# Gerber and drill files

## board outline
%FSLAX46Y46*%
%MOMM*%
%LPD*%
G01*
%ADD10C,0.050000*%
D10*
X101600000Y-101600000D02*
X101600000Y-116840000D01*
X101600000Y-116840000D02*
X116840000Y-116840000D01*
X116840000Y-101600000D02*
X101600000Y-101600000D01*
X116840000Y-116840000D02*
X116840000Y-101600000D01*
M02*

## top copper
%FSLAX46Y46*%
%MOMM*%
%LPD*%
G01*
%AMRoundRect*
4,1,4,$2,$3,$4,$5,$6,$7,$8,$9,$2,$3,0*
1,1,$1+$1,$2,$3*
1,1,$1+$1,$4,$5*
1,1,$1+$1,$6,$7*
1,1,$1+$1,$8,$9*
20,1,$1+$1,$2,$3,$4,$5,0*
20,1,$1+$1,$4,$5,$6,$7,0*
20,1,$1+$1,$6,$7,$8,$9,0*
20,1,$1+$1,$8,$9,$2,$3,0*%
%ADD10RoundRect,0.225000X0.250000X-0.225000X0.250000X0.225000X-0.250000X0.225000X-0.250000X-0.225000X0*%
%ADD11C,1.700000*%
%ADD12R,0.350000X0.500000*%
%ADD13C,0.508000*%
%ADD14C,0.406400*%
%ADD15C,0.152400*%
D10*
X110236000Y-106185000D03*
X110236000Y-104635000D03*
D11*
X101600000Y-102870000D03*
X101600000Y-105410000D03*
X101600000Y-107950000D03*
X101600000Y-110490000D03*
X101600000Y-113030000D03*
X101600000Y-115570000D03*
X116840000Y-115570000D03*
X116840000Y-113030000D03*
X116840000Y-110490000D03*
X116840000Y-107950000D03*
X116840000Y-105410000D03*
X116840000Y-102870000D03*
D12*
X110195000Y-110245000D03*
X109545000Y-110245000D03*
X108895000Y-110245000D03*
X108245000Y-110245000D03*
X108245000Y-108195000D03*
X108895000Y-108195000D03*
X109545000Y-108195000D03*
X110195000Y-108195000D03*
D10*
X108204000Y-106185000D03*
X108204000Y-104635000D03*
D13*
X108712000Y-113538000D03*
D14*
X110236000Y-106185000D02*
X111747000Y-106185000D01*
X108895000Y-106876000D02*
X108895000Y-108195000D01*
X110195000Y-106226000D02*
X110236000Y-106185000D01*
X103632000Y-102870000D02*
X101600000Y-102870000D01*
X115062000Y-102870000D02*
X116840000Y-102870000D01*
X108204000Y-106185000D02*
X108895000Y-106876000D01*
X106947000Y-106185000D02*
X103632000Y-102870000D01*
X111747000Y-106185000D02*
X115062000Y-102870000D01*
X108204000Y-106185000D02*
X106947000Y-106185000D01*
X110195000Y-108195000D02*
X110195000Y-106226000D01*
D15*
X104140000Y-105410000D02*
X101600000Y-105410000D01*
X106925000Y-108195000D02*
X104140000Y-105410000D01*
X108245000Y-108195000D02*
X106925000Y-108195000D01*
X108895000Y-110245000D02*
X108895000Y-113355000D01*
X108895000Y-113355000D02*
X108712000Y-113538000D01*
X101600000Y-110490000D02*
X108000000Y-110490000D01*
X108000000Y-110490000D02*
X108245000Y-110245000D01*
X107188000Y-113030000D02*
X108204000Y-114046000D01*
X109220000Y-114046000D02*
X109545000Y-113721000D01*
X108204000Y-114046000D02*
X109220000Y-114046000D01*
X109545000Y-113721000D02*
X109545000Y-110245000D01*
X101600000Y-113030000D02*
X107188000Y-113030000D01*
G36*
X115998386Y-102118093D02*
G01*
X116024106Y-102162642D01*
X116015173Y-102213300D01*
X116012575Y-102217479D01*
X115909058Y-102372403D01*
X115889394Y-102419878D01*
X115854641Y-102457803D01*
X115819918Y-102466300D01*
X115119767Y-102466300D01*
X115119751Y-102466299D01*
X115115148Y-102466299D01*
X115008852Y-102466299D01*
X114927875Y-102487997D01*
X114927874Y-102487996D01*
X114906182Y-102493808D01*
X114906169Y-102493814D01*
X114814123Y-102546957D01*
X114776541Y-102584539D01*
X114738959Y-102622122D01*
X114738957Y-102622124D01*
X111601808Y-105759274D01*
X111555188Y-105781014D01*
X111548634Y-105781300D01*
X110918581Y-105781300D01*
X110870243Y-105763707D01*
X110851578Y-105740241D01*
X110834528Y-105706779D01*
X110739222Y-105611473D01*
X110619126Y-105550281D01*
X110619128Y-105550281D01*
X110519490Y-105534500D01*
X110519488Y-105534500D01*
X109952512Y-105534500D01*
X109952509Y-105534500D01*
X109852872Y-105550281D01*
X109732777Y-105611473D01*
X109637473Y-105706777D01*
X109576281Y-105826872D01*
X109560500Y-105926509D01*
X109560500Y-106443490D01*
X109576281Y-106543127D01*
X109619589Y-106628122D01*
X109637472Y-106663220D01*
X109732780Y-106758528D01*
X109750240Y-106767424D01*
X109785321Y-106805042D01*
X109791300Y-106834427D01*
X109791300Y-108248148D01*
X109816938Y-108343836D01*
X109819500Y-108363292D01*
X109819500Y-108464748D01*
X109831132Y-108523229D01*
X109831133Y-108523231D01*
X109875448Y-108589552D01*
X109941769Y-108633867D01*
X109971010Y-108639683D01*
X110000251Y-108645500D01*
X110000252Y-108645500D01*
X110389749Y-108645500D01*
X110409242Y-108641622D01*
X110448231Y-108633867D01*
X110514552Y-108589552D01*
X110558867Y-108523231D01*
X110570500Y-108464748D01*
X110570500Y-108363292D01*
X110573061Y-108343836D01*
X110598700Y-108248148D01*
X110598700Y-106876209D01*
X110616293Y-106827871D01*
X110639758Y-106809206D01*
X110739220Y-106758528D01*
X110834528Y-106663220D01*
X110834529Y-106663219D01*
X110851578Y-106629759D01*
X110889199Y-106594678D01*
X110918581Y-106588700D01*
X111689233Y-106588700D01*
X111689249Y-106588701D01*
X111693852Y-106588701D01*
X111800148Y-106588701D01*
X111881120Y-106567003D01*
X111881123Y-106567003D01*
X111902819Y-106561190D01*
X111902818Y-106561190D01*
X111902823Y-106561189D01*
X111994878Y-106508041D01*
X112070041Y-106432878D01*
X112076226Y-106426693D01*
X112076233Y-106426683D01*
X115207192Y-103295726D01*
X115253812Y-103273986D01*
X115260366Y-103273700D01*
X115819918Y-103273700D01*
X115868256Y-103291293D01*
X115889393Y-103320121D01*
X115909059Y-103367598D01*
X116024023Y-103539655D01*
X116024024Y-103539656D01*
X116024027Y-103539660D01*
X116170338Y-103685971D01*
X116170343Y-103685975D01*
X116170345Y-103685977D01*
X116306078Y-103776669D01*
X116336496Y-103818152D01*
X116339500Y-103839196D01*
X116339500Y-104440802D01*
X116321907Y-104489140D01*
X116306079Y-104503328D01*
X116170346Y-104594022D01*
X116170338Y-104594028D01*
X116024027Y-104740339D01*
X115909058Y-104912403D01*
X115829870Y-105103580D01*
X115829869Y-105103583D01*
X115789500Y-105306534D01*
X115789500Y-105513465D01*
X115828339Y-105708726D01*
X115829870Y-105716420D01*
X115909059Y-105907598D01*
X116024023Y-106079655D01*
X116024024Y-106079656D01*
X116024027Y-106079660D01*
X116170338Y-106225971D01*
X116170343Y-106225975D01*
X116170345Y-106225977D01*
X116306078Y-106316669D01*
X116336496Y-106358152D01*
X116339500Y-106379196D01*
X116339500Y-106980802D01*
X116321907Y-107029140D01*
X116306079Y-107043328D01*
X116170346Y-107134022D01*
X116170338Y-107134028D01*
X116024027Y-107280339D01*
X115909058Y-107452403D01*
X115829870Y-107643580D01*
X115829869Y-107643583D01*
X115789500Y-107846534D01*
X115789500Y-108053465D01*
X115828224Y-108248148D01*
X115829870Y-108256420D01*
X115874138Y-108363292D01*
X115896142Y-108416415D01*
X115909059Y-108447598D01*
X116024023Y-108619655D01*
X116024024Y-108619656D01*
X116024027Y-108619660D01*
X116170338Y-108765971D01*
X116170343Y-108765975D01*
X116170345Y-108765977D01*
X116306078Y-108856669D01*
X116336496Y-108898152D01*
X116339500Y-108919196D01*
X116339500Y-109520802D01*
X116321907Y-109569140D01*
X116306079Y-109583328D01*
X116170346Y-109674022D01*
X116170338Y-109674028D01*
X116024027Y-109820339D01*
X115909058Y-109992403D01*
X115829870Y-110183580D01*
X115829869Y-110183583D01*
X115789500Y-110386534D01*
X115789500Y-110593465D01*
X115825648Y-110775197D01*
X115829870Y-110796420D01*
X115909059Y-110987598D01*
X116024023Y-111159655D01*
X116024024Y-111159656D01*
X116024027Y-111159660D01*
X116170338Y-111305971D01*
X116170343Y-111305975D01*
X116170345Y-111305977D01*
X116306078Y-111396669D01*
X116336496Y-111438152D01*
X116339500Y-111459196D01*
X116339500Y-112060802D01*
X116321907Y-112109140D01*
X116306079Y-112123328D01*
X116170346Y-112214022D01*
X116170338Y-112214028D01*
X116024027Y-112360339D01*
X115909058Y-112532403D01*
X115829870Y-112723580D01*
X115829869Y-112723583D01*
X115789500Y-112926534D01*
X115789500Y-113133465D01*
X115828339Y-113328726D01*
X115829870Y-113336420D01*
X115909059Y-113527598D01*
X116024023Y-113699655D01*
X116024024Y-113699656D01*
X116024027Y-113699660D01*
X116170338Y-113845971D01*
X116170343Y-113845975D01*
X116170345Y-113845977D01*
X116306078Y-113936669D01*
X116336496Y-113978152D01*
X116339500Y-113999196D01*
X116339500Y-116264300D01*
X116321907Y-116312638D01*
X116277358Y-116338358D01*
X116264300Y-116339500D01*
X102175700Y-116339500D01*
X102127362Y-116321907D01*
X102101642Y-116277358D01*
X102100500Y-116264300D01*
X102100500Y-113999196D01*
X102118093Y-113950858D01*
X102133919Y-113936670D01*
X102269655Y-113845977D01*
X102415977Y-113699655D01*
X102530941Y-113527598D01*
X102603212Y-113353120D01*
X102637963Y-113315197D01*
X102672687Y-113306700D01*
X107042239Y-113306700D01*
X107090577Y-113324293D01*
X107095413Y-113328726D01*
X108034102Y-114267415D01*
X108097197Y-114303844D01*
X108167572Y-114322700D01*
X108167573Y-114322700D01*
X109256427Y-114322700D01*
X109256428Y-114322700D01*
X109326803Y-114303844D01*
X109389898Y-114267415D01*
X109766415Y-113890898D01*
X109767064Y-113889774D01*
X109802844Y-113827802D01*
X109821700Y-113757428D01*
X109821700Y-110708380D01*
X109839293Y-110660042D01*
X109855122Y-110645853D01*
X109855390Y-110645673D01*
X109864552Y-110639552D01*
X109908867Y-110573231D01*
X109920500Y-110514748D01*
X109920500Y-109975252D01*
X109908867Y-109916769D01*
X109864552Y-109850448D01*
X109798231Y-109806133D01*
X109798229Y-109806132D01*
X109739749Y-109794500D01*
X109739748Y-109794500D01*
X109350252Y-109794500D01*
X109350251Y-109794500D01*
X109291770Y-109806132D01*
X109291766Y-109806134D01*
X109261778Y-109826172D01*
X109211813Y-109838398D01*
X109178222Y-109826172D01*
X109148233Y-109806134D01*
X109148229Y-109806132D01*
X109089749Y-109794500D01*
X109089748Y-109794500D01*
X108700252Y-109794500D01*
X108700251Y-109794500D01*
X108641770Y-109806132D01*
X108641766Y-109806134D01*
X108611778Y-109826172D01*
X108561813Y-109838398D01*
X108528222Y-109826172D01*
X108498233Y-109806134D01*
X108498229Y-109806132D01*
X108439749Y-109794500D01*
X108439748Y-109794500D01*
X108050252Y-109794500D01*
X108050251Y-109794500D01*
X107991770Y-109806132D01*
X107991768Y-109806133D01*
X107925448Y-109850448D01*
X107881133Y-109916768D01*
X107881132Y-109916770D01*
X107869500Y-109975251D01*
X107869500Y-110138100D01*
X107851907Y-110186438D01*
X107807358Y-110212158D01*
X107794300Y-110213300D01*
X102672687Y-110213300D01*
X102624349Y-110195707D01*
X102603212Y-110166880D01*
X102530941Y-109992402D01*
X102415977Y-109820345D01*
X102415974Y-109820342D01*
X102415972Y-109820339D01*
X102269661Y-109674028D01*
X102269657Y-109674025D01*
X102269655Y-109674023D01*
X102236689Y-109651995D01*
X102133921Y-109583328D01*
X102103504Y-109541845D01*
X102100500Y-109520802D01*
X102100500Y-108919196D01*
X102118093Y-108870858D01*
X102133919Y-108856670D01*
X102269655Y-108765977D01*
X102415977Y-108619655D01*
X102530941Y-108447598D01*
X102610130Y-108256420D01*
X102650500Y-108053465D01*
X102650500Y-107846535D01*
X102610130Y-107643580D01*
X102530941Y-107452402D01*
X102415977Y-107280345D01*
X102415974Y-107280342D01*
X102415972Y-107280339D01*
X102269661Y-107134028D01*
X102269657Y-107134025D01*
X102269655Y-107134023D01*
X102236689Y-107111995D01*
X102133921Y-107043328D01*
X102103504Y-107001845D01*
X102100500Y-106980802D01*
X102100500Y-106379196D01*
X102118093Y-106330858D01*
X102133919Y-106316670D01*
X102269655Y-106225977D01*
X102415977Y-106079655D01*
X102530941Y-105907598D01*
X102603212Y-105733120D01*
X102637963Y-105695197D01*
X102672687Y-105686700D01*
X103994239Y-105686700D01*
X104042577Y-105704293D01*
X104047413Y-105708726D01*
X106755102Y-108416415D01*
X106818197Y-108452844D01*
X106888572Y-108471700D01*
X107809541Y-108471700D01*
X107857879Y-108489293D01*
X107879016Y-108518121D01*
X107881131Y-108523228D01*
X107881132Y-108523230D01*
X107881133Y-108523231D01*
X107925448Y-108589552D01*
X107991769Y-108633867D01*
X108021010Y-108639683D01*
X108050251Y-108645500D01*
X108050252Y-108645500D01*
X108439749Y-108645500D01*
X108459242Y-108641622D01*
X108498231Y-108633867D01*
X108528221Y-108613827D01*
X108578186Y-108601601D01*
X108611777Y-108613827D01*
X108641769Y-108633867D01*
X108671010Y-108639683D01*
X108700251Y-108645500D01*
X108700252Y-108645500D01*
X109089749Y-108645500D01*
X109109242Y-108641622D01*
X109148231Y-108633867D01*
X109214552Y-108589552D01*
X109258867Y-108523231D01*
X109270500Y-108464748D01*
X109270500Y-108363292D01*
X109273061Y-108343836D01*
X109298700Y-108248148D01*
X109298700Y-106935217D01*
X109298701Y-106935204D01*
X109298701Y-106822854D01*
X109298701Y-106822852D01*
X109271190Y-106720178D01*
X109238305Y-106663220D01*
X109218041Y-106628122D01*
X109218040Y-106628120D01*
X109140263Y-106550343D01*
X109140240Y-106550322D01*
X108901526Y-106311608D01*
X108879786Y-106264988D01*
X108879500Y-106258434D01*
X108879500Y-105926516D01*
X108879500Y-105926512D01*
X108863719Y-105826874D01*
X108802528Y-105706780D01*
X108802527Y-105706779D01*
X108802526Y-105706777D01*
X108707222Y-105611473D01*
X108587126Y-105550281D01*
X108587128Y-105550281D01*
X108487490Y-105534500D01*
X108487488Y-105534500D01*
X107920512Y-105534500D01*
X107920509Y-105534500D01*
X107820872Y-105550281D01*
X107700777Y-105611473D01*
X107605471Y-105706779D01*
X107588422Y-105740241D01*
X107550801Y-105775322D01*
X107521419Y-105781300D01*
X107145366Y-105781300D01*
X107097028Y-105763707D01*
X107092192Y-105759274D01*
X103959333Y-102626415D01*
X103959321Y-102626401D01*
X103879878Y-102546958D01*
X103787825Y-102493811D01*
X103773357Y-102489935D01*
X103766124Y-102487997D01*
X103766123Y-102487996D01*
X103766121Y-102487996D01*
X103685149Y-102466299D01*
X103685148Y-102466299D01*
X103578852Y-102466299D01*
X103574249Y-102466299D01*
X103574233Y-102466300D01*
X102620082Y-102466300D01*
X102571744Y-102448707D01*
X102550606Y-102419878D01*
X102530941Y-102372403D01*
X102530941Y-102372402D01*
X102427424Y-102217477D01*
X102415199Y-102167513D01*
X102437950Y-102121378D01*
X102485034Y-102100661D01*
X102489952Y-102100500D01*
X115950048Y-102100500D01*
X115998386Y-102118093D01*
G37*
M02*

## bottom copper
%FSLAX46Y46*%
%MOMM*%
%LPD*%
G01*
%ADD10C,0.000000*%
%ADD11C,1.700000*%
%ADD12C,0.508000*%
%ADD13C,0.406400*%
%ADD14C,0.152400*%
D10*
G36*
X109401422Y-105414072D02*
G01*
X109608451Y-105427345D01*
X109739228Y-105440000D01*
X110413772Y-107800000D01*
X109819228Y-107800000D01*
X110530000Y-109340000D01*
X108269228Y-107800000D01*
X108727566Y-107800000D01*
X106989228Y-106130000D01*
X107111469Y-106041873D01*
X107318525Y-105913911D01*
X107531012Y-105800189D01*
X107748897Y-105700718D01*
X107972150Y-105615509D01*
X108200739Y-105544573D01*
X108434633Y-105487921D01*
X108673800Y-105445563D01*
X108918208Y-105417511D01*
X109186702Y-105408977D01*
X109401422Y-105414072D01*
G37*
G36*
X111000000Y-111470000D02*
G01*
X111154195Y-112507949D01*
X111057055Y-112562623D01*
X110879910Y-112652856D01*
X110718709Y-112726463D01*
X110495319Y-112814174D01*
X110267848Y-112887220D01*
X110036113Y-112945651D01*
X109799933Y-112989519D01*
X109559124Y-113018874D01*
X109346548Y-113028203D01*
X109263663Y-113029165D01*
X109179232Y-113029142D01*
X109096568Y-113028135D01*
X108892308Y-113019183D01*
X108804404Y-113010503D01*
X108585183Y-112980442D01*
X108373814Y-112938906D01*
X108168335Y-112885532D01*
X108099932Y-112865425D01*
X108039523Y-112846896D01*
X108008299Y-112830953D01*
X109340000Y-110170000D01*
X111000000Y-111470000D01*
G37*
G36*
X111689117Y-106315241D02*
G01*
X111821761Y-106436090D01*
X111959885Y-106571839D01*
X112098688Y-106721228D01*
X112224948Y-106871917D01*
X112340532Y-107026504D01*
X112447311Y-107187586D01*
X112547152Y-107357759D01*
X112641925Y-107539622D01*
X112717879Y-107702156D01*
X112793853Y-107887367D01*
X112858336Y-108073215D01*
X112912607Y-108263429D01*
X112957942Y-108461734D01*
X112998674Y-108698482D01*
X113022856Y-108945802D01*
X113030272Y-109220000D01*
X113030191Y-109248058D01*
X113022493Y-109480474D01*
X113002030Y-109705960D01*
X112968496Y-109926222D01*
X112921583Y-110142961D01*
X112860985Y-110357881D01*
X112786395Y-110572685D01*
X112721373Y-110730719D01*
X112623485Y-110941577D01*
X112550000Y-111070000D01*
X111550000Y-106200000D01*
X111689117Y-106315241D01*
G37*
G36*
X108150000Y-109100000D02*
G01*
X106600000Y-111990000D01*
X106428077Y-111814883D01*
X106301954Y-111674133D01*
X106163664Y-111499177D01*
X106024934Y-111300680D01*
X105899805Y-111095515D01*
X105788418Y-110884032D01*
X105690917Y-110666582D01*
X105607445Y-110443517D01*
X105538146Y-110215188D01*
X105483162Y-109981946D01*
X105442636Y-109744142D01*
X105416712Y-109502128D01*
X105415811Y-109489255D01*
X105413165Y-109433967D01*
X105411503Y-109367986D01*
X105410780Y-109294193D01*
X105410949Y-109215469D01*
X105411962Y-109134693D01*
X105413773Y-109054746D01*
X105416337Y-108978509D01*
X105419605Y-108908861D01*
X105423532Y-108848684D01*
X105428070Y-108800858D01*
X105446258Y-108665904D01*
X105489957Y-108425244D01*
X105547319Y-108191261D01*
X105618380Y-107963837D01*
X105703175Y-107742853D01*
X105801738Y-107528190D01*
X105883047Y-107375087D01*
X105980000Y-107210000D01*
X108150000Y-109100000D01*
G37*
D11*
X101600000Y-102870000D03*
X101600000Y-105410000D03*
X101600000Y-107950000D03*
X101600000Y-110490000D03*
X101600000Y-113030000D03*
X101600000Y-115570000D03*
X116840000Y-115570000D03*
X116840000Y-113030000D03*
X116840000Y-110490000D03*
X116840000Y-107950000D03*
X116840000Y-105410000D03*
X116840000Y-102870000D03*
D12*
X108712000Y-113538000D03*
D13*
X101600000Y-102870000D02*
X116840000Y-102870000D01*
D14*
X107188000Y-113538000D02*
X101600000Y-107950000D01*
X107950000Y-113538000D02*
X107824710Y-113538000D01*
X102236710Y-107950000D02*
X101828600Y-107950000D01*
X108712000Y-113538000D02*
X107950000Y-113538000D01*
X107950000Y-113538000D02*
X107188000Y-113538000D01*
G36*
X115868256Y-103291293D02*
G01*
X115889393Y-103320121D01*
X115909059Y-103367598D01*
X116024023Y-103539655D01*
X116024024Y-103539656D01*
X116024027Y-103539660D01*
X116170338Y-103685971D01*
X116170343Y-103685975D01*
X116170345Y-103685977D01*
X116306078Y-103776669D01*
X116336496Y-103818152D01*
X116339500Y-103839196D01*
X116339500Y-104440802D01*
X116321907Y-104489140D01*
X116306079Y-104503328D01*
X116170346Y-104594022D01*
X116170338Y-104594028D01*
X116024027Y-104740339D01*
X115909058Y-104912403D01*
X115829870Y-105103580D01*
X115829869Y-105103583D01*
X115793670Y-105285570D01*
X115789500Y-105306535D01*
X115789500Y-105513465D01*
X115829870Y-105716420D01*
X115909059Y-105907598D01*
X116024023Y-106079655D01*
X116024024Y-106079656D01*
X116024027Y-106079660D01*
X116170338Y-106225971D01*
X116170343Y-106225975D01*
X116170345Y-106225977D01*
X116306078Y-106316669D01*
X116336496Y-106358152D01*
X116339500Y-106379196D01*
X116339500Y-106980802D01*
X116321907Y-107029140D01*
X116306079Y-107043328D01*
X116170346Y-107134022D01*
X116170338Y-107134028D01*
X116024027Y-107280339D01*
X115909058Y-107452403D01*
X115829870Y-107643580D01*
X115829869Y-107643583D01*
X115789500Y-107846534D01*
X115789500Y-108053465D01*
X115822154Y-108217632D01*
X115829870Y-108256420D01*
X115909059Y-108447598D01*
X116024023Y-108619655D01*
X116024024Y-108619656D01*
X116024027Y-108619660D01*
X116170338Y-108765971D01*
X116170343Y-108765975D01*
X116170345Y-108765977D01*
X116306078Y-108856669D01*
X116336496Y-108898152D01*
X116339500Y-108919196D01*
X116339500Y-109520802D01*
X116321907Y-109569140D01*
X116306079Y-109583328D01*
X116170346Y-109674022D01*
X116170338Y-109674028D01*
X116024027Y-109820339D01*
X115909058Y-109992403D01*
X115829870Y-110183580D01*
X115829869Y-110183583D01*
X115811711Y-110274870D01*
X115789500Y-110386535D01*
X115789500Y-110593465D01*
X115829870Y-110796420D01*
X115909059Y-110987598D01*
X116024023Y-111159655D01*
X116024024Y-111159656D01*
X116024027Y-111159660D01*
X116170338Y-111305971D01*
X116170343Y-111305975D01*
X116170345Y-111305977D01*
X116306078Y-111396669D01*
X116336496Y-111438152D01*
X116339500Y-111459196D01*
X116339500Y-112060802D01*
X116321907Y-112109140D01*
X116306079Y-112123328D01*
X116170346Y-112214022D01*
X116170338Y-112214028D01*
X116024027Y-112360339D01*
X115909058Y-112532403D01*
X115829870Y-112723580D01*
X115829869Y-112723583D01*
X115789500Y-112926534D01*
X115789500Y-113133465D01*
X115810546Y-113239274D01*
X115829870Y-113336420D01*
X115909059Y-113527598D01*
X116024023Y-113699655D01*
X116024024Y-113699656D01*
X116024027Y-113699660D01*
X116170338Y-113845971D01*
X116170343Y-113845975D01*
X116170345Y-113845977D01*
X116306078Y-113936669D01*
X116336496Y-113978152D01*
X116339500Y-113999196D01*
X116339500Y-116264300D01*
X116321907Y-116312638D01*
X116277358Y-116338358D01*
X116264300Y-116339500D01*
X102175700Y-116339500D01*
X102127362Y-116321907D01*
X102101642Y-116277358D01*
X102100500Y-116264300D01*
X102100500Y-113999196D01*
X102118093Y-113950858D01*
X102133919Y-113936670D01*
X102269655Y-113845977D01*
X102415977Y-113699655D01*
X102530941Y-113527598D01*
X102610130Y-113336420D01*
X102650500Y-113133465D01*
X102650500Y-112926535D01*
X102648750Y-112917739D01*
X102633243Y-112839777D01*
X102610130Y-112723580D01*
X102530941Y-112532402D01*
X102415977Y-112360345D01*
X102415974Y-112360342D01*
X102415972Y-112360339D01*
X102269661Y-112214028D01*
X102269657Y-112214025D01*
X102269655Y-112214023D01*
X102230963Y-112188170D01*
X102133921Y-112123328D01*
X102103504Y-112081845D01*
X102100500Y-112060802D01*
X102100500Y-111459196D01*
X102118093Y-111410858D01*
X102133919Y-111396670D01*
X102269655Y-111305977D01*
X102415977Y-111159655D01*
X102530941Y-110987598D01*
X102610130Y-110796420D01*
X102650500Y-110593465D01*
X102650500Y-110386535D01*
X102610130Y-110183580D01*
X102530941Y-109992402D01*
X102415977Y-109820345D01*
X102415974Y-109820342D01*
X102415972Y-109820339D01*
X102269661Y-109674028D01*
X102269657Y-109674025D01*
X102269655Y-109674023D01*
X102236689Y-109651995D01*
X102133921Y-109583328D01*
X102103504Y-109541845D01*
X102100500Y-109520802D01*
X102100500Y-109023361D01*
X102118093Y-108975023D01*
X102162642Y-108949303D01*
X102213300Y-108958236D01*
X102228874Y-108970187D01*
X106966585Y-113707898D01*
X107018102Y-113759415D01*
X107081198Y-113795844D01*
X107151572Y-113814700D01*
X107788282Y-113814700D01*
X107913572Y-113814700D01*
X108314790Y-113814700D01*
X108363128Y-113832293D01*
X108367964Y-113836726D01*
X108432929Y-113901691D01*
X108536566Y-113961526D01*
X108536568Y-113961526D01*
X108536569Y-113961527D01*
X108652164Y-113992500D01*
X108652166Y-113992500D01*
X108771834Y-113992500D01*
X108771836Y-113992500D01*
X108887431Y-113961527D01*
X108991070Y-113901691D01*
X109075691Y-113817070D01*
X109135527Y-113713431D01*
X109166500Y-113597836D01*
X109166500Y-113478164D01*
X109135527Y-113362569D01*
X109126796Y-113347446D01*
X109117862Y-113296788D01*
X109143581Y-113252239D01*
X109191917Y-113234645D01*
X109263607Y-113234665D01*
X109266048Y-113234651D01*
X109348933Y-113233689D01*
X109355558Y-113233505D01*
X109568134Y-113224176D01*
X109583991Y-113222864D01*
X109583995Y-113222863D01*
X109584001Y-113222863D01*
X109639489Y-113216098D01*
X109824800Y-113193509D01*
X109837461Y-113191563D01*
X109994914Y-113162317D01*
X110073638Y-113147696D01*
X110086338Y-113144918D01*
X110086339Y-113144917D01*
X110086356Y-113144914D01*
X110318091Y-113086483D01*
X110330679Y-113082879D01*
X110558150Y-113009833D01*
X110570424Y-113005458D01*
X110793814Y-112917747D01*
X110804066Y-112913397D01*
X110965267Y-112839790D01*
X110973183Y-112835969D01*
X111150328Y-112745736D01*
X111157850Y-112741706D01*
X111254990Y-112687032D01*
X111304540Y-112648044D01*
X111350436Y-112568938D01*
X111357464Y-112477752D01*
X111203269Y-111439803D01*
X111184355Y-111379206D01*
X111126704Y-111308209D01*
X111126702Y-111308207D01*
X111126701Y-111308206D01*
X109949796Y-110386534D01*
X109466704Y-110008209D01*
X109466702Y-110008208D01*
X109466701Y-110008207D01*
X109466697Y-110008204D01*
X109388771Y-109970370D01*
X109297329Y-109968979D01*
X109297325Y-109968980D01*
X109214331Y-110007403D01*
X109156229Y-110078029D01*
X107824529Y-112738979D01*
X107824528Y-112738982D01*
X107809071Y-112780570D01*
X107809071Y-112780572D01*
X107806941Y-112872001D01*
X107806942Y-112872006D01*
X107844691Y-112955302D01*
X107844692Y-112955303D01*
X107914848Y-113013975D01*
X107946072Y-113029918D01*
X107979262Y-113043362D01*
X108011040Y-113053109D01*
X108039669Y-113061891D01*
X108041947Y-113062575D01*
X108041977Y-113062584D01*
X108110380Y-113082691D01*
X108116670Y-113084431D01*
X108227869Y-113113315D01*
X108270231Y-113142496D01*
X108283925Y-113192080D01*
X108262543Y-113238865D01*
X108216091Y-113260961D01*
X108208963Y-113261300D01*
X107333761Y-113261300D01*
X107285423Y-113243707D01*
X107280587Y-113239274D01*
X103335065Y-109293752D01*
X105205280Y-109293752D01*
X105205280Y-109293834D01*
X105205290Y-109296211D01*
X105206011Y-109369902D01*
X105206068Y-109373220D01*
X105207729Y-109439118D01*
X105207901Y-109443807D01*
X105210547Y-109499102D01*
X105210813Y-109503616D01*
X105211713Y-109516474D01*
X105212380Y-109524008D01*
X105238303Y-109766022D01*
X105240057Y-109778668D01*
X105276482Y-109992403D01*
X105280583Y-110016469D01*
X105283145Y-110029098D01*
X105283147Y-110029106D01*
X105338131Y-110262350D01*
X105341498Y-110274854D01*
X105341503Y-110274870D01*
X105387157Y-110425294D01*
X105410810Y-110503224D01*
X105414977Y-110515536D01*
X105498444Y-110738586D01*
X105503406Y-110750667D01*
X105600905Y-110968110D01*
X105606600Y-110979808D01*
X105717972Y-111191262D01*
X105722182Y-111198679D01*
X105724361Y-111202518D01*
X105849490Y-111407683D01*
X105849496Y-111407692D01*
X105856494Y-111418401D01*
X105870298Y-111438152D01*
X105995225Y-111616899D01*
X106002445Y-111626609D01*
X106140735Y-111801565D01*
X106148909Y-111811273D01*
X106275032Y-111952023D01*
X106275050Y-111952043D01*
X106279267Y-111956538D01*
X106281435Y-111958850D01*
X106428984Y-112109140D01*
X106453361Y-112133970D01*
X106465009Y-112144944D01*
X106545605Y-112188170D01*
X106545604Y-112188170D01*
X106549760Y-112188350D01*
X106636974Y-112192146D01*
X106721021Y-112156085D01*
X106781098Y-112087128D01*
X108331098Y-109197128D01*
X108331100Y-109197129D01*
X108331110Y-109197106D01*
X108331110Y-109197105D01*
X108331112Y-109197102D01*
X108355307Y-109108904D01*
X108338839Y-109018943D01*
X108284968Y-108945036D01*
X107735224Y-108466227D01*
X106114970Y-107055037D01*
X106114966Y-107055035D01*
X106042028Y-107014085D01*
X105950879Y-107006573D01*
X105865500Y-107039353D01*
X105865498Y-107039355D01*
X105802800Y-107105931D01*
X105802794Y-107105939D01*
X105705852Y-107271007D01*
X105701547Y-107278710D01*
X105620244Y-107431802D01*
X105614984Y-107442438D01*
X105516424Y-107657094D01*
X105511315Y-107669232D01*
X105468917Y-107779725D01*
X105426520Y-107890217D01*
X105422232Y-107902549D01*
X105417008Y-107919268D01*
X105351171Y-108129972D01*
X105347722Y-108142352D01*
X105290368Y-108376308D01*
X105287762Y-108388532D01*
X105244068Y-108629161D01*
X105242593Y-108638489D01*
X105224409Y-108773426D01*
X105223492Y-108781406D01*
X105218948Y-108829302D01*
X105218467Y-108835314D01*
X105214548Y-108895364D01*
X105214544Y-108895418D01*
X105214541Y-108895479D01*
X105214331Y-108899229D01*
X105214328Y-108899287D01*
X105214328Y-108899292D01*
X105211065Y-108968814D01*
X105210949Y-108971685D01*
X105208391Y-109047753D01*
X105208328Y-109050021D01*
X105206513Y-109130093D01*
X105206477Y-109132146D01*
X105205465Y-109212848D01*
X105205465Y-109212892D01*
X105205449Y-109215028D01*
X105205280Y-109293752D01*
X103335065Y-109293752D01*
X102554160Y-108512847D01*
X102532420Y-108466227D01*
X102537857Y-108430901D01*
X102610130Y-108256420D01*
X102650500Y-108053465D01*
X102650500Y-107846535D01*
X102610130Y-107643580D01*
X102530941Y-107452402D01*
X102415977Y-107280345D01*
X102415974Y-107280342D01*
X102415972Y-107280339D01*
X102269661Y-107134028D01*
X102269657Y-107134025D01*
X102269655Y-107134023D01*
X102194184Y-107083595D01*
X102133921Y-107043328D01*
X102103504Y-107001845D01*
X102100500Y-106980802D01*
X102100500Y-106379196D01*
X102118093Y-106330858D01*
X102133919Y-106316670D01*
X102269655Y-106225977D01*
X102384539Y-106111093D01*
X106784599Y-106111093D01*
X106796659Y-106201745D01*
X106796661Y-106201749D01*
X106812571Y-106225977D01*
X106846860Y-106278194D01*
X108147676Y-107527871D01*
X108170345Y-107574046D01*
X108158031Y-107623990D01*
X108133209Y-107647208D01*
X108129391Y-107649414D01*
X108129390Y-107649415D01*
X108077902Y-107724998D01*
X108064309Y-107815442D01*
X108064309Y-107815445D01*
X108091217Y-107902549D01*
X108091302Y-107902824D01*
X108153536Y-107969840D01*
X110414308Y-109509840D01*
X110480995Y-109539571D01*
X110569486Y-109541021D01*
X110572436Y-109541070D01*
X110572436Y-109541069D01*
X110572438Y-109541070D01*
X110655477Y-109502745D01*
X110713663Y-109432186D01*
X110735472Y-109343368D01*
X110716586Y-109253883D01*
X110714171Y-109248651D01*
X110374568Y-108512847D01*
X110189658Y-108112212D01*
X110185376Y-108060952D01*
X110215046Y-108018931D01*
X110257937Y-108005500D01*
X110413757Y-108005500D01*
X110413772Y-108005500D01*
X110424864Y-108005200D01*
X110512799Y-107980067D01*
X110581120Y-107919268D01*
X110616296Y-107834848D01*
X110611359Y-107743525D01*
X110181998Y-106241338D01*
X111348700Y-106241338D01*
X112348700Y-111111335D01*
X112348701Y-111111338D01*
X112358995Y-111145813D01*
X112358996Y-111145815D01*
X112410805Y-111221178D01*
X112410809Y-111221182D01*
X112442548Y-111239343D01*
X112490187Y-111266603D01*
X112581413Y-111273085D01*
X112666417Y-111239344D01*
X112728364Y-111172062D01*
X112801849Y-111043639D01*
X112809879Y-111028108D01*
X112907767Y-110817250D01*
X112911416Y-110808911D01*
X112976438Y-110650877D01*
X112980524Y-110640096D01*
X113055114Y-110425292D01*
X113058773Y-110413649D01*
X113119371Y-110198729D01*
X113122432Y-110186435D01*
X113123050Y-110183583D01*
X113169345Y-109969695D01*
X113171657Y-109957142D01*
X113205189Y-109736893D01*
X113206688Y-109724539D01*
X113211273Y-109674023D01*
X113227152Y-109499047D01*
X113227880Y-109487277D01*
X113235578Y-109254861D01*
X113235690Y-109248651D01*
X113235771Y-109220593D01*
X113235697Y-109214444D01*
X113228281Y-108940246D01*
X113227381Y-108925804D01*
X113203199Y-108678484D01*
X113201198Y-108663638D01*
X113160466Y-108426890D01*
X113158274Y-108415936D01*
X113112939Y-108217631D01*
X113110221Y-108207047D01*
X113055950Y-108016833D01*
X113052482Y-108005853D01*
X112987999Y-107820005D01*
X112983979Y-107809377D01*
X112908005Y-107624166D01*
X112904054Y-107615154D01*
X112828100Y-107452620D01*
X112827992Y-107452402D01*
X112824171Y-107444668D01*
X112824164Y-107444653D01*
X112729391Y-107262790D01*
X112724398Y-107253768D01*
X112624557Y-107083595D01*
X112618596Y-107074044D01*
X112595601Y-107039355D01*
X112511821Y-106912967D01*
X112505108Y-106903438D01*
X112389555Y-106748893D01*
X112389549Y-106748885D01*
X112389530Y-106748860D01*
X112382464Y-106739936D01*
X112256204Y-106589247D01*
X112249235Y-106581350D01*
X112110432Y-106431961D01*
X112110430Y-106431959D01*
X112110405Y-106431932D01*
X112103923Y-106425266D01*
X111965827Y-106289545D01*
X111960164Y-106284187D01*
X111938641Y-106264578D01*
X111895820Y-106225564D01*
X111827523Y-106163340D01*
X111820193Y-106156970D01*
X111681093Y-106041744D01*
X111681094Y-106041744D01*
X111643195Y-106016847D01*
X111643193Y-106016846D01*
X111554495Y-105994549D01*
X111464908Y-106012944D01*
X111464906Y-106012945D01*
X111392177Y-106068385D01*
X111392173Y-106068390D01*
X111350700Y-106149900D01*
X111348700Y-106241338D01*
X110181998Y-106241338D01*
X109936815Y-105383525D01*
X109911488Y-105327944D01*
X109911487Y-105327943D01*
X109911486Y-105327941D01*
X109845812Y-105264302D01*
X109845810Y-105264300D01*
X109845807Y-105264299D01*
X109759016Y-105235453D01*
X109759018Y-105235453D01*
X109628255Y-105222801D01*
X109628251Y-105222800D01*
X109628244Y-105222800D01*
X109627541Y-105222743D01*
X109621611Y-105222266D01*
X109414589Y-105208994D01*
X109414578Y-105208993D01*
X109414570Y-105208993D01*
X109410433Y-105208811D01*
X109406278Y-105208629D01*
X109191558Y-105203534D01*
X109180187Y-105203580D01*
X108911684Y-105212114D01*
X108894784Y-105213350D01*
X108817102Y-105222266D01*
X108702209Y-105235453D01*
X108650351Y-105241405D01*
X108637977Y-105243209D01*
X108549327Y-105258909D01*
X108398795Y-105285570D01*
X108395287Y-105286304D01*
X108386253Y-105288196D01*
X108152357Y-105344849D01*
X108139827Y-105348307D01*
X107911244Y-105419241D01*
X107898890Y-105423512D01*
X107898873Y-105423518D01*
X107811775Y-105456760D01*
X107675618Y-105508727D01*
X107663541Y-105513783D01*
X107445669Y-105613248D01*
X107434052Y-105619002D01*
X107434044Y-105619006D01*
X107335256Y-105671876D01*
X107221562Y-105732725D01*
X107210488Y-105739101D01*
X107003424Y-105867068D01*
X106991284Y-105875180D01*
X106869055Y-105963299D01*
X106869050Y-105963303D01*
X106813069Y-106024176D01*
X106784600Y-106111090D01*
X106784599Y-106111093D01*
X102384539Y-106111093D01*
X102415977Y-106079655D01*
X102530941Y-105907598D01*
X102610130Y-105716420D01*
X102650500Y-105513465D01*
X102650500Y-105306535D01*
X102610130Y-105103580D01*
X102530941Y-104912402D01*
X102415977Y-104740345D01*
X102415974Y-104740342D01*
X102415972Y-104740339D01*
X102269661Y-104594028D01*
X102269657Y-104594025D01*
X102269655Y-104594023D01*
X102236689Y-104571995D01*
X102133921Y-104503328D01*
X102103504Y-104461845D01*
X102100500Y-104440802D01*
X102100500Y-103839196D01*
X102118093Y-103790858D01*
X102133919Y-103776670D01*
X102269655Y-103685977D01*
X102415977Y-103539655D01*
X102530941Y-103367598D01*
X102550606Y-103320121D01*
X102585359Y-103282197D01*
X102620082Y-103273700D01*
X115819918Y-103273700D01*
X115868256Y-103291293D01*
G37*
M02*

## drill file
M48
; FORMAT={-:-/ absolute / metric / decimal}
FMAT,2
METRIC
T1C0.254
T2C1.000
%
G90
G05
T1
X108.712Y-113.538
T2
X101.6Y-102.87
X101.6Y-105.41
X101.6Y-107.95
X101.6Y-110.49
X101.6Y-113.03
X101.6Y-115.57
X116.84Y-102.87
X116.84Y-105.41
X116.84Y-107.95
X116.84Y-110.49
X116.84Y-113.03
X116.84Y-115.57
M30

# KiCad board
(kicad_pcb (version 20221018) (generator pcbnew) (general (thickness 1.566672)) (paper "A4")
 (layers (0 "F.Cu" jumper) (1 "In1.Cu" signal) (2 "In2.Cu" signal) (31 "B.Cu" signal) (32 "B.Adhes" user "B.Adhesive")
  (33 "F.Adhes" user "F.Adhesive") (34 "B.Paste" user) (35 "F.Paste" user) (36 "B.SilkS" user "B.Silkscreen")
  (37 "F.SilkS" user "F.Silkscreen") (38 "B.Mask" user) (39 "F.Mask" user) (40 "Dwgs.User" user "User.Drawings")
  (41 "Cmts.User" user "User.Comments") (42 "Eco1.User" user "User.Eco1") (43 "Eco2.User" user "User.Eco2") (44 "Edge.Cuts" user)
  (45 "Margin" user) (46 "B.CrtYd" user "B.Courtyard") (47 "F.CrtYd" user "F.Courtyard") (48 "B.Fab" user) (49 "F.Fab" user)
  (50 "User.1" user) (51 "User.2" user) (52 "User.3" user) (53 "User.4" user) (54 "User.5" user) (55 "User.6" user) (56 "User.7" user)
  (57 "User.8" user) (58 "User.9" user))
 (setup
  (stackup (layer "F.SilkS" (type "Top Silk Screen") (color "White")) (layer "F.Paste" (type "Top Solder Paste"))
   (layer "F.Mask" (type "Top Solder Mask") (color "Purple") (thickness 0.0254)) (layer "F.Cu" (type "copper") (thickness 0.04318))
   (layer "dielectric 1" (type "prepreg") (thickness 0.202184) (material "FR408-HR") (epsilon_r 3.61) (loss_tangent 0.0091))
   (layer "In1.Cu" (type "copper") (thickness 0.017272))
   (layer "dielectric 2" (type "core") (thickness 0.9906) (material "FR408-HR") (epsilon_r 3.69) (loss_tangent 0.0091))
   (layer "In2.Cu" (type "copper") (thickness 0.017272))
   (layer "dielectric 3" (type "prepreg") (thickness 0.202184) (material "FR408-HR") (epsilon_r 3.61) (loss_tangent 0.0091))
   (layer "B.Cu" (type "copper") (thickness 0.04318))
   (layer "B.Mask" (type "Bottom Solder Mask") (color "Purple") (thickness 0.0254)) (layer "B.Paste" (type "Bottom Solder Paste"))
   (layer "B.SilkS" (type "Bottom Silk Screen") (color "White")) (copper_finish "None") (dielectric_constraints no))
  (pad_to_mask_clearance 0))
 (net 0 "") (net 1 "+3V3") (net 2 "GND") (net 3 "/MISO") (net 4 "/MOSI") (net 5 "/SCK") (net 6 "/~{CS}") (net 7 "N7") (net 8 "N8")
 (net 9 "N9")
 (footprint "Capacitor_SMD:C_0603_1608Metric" (layer "F.Cu") (at 110.236 105.41 90)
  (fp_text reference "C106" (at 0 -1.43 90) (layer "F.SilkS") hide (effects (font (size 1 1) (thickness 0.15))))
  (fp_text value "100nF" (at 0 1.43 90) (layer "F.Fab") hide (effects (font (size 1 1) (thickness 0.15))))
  (pad "1" smd roundrect (at -0.775 0 90) (size 0.9 0.95) (layers "F.Cu" "F.Paste" "F.Mask") (roundrect_rratio 0.25) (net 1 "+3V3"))
  (pad "2" smd roundrect (at 0.775 0 90) (size 0.9 0.95) (layers "F.Cu" "F.Paste" "F.Mask") (roundrect_rratio 0.25) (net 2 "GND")))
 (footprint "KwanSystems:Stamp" (layer "F.Cu") (at 109.22 109.22)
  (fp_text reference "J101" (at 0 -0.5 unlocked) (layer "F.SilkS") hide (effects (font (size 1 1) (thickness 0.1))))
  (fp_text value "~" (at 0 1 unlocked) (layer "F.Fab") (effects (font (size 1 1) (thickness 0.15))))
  (fp_line (start -7.62 -7.62) (end -7.62 7.62) (stroke (width 0.05) (type default)) (layer "Edge.Cuts"))
  (fp_line (start -7.62 7.62) (end 7.62 7.62) (stroke (width 0.05) (type default)) (layer "Edge.Cuts"))
  (fp_line (start 7.62 -7.62) (end -7.62 -7.62) (stroke (width 0.05) (type default)) (layer "Edge.Cuts"))
  (fp_line (start 7.62 7.62) (end 7.62 -7.62) (stroke (width 0.05) (type default)) (layer "Edge.Cuts"))
  (pad "1" thru_hole circle (at -7.62 -6.35) (size 1.7 1.7) (drill 1) (layers "*.Cu" "*.Mask") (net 1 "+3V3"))
  (pad "2" thru_hole circle (at -7.62 -3.81) (size 1.7 1.7) (drill 1) (layers "*.Cu" "*.Mask") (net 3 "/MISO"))
  (pad "3" thru_hole circle (at -7.62 -1.27) (size 1.7 1.7) (drill 1) (layers "*.Cu" "*.Mask") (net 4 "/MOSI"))
  (pad "4" thru_hole circle (at -7.62 1.27) (size 1.7 1.7) (drill 1) (layers "*.Cu" "*.Mask") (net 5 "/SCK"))
  (pad "5" thru_hole circle (at -7.62 3.81) (size 1.7 1.7) (drill 1) (layers "*.Cu" "*.Mask") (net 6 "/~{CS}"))
  (pad "6" thru_hole circle (at -7.62 6.35) (size 1.7 1.7) (drill 1) (layers "*.Cu" "*.Mask") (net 2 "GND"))
  (pad "7" thru_hole circle (at 7.62 6.35) (size 1.7 1.7) (drill 1) (layers "*.Cu" "*.Mask") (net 2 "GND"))
  (pad "8" thru_hole circle (at 7.62 3.81) (size 1.7 1.7) (drill 1) (layers "*.Cu" "*.Mask") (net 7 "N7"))
  (pad "9" thru_hole circle (at 7.62 1.27) (size 1.7 1.7) (drill 1) (layers "*.Cu" "*.Mask") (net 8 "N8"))
  (pad "10" thru_hole circle (at 7.62 -1.27) (size 1.7 1.7) (drill 1) (layers "*.Cu" "*.Mask"))
  (pad "11" thru_hole circle (at 7.62 -3.81) (size 1.7 1.7) (drill 1) (layers "*.Cu" "*.Mask") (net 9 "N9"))
  (pad "12" thru_hole circle (at 7.62 -6.35) (size 1.7 1.7) (drill 1) (layers "*.Cu" "*.Mask") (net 1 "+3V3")))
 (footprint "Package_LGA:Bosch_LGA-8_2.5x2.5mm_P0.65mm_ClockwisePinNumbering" (layer "F.Cu") (at 109.22 109.22 180)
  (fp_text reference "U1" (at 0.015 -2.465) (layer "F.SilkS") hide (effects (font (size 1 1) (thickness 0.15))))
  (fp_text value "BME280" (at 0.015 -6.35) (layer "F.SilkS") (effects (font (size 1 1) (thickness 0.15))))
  (pad "1" smd rect (at -0.975 -1.025 270) (size 0.5 0.35) (layers "F.Cu" "F.Paste" "F.Mask") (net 2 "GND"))
  (pad "2" smd rect (at -0.325 -1.025 270) (size 0.5 0.35) (layers "F.Cu" "F.Paste" "F.Mask") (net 6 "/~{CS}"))
  (pad "3" smd rect (at 0.325 -1.025 270) (size 0.5 0.35) (layers "F.Cu" "F.Paste" "F.Mask") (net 4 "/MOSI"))
  (pad "4" smd rect (at 0.975 -1.025 270) (size 0.5 0.35) (layers "F.Cu" "F.Paste" "F.Mask") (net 5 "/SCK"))
  (pad "5" smd rect (at 0.975 1.025 270) (size 0.5 0.35) (layers "F.Cu" "F.Paste" "F.Mask") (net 3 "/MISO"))
  (pad "6" smd rect (at 0.325 1.025 270) (size 0.5 0.35) (layers "F.Cu" "F.Paste" "F.Mask") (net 1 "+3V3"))
  (pad "7" smd rect (at -0.325 1.025 270) (size 0.5 0.35) (layers "F.Cu" "F.Paste" "F.Mask") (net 2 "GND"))
  (pad "8" smd rect (at -0.975 1.025 270) (size 0.5 0.35) (layers "F.Cu" "F.Paste" "F.Mask") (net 1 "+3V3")))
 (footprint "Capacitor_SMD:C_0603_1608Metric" (layer "F.Cu") (at 108.204 105.41 90)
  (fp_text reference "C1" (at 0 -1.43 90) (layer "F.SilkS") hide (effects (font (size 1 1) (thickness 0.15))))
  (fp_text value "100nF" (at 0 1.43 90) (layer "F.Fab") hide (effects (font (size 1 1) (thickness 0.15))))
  (pad "1" smd roundrect (at -0.775 0 90) (size 0.9 0.95) (layers "F.Cu" "F.Paste" "F.Mask") (roundrect_rratio 0.25) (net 1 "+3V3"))
  (pad "2" smd roundrect (at 0.775 0 90) (size 0.9 0.95) (layers "F.Cu" "F.Paste" "F.Mask") (roundrect_rratio 0.25) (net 2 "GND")))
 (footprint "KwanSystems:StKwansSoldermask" (layer "B.Cu") (at 109.22 109.22 180)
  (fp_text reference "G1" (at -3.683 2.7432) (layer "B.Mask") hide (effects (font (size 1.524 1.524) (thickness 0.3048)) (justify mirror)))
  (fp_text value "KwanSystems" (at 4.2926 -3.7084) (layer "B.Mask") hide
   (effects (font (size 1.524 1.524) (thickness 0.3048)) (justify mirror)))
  (fp_poly
   (pts (xy 0.301792 3.802489) (xy 0.5462 3.774437) (xy 0.785367 3.732079) (xy 1.019261 3.675427) (xy 1.24785 3.604491)
    (xy 1.471103 3.519282) (xy 1.688988 3.419811) (xy 1.901475 3.306089) (xy 2.108531 3.178127) (xy 2.230772 3.09) (xy 0.492434 1.42)
    (xy 0.950772 1.42) (xy -1.31 -0.12) (xy -0.599228 1.42) (xy -1.193772 1.42) (xy -0.519228 3.78) (xy -0.388451 3.792655)
    (xy -0.181422 3.805928) (xy 0.033298 3.811023))
   (stroke (width 0) (type solid)) (fill solid) (layer "B.Cu"))
  (fp_poly
   (pts (xy 1.211701 -3.610953) (xy 1.180477 -3.626896) (xy 1.120068 -3.645425) (xy 1.051665 -3.665532) (xy 0.846186 -3.718906)
    (xy 0.634817 -3.760442) (xy 0.415596 -3.790503) (xy 0.327692 -3.799183) (xy 0.123432 -3.808135) (xy 0.040768 -3.809142)
    (xy -0.043663 -3.809165) (xy -0.126548 -3.808203) (xy -0.339124 -3.798874) (xy -0.579933 -3.769519) (xy -0.816113 -3.725651)
    (xy -1.047848 -3.66722) (xy -1.275319 -3.594174) (xy -1.498709 -3.506463) (xy -1.65991 -3.432856) (xy -1.837055 -3.342623)
    (xy -1.934195 -3.287949) (xy -1.78 -2.25) (xy -0.12 -0.95))
   (stroke (width 0) (type solid)) (fill solid) (layer "B.Cu"))
  (fp_poly
   (pts (xy -3.33 -1.85) (xy -3.403485 -1.721577) (xy -3.501373 -1.510719) (xy -3.566395 -1.352685) (xy -3.640985 -1.137881)
    (xy -3.701583 -0.922961) (xy -3.748496 -0.706222) (xy -3.78203 -0.48596) (xy -3.802493 -0.260474) (xy -3.810191 -0.028058)
    (xy -3.810272 0) (xy -3.802856 0.274198) (xy -3.778674 0.521518) (xy -3.737942 0.758266) (xy -3.692607 0.956571) (xy -3.638336 1.146785)
    (xy -3.573853 1.332633) (xy -3.497879 1.517844) (xy -3.421925 1.680378) (xy -3.327152 1.862241) (xy -3.227311 2.032414)
    (xy -3.120532 2.193496) (xy -3.004948 2.348083) (xy -2.878688 2.498772) (xy -2.739885 2.648161) (xy -2.601761 2.78391)
    (xy -2.469117 2.904759) (xy -2.33 3.02))
   (stroke (width 0) (type solid)) (fill solid) (layer "B.Cu"))
  (fp_poly
   (pts (xy 3.336953 1.844913) (xy 3.418262 1.69181) (xy 3.516825 1.477147) (xy 3.60162 1.256163) (xy 3.672681 1.028739)
    (xy 3.730043 0.794756) (xy 3.773742 0.554096) (xy 3.79193 0.419142) (xy 3.796468 0.371316) (xy 3.800395 0.311139) (xy 3.803663 0.241491)
    (xy 3.806227 0.165254) (xy 3.808038 0.085307) (xy 3.809051 0.004531) (xy 3.80922 -0.074193) (xy 3.808497 -0.147986)
    (xy 3.806835 -0.213967) (xy 3.804189 -0.269255) (xy 3.803288 -0.282128) (xy 3.777364 -0.524142) (xy 3.736838 -0.761946)
    (xy 3.681854 -0.995188) (xy 3.612555 -1.223517) (xy 3.529083 -1.446582) (xy 3.431582 -1.664032) (xy 3.320195 -1.875515)
    (xy 3.195066 -2.08068) (xy 3.056336 -2.279177) (xy 2.918046 -2.454133) (xy 2.791923 -2.594883) (xy 2.62 -2.77) (xy 1.07 0.12)
    (xy 3.24 2.01))
   (stroke (width 0) (type solid)) (fill solid) (layer "B.Cu")))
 (segment (start 110.236 106.185) (end 111.747 106.185) (width 0.4064) (layer "F.Cu") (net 1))
 (segment (start 108.895 106.876) (end 108.895 108.195) (width 0.4064) (layer "F.Cu") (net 1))
 (segment (start 110.195 106.226) (end 110.236 106.185) (width 0.4064) (layer "F.Cu") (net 1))
 (segment (start 103.632 102.87) (end 101.6 102.87) (width 0.4064) (layer "F.Cu") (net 1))
 (segment (start 115.062 102.87) (end 116.84 102.87) (width 0.4064) (layer "F.Cu") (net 1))
 (segment (start 108.204 106.185) (end 108.895 106.876) (width 0.4064) (layer "F.Cu") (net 1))
 (segment (start 106.947 106.185) (end 103.632 102.87) (width 0.4064) (layer "F.Cu") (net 1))
 (segment (start 111.747 106.185) (end 115.062 102.87) (width 0.4064) (layer "F.Cu") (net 1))
 (segment (start 108.204 106.185) (end 106.947 106.185) (width 0.4064) (layer "F.Cu") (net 1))
 (segment (start 110.195 108.195) (end 110.195 106.226) (width 0.4064) (layer "F.Cu") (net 1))
 (segment (start 101.6 102.87) (end 116.84 102.87) (width 0.4064) (layer "B.Cu") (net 1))
 (segment (start 104.14 105.41) (end 101.6 105.41) (width 0.1524) (layer "F.Cu") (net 3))
 (segment (start 106.925 108.195) (end 104.14 105.41) (width 0.1524) (layer "F.Cu") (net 3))
 (segment (start 108.245 108.195) (end 106.925 108.195) (width 0.1524) (layer "F.Cu") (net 3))
 (segment (start 108.895 110.245) (end 108.895 113.355) (width 0.1524) (layer "F.Cu") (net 4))
 (segment (start 108.895 113.355) (end 108.712 113.538) (width 0.1524) (layer "F.Cu") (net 4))
 (via (at 108.712 113.538) (size 0.508) (drill 0.254) (layers "F.Cu" "B.Cu") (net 4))
 (segment (start 107.188 113.538) (end 101.6 107.95) (width 0.1524) (layer "B.Cu") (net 4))
 (segment (start 107.95 113.538) (end 107.82471 113.538) (width 0.1524) (layer "B.Cu") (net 4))
 (segment (start 102.23671 107.95) (end 101.8286 107.95) (width 0.1524) (layer "B.Cu") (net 4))
 (segment (start 108.712 113.538) (end 107.95 113.538) (width 0.1524) (layer "B.Cu") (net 4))
 (segment (start 107.95 113.538) (end 107.188 113.538) (width 0.1524) (layer "B.Cu") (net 4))
 (segment (start 101.6 110.49) (end 108 110.49) (width 0.1524) (layer "F.Cu") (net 5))
 (segment (start 108 110.49) (end 108.245 110.245) (width 0.1524) (layer "F.Cu") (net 5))
 (segment (start 107.188 113.03) (end 108.204 114.046) (width 0.1524) (layer "F.Cu") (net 6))
 (segment (start 109.22 114.046) (end 109.545 113.721) (width 0.1524) (layer "F.Cu") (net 6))
 (segment (start 108.204 114.046) (end 109.22 114.046) (width 0.1524) (layer "F.Cu") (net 6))
 (segment (start 109.545 113.721) (end 109.545 110.245) (width 0.1524) (layer "F.Cu") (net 6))
 (segment (start 101.6 113.03) (end 107.188 113.03) (width 0.1524) (layer "F.Cu") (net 6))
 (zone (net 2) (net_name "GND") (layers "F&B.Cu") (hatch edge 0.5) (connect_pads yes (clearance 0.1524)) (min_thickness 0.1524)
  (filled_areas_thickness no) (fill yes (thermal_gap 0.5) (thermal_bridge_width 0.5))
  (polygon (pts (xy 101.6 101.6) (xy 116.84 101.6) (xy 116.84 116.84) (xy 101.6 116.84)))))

